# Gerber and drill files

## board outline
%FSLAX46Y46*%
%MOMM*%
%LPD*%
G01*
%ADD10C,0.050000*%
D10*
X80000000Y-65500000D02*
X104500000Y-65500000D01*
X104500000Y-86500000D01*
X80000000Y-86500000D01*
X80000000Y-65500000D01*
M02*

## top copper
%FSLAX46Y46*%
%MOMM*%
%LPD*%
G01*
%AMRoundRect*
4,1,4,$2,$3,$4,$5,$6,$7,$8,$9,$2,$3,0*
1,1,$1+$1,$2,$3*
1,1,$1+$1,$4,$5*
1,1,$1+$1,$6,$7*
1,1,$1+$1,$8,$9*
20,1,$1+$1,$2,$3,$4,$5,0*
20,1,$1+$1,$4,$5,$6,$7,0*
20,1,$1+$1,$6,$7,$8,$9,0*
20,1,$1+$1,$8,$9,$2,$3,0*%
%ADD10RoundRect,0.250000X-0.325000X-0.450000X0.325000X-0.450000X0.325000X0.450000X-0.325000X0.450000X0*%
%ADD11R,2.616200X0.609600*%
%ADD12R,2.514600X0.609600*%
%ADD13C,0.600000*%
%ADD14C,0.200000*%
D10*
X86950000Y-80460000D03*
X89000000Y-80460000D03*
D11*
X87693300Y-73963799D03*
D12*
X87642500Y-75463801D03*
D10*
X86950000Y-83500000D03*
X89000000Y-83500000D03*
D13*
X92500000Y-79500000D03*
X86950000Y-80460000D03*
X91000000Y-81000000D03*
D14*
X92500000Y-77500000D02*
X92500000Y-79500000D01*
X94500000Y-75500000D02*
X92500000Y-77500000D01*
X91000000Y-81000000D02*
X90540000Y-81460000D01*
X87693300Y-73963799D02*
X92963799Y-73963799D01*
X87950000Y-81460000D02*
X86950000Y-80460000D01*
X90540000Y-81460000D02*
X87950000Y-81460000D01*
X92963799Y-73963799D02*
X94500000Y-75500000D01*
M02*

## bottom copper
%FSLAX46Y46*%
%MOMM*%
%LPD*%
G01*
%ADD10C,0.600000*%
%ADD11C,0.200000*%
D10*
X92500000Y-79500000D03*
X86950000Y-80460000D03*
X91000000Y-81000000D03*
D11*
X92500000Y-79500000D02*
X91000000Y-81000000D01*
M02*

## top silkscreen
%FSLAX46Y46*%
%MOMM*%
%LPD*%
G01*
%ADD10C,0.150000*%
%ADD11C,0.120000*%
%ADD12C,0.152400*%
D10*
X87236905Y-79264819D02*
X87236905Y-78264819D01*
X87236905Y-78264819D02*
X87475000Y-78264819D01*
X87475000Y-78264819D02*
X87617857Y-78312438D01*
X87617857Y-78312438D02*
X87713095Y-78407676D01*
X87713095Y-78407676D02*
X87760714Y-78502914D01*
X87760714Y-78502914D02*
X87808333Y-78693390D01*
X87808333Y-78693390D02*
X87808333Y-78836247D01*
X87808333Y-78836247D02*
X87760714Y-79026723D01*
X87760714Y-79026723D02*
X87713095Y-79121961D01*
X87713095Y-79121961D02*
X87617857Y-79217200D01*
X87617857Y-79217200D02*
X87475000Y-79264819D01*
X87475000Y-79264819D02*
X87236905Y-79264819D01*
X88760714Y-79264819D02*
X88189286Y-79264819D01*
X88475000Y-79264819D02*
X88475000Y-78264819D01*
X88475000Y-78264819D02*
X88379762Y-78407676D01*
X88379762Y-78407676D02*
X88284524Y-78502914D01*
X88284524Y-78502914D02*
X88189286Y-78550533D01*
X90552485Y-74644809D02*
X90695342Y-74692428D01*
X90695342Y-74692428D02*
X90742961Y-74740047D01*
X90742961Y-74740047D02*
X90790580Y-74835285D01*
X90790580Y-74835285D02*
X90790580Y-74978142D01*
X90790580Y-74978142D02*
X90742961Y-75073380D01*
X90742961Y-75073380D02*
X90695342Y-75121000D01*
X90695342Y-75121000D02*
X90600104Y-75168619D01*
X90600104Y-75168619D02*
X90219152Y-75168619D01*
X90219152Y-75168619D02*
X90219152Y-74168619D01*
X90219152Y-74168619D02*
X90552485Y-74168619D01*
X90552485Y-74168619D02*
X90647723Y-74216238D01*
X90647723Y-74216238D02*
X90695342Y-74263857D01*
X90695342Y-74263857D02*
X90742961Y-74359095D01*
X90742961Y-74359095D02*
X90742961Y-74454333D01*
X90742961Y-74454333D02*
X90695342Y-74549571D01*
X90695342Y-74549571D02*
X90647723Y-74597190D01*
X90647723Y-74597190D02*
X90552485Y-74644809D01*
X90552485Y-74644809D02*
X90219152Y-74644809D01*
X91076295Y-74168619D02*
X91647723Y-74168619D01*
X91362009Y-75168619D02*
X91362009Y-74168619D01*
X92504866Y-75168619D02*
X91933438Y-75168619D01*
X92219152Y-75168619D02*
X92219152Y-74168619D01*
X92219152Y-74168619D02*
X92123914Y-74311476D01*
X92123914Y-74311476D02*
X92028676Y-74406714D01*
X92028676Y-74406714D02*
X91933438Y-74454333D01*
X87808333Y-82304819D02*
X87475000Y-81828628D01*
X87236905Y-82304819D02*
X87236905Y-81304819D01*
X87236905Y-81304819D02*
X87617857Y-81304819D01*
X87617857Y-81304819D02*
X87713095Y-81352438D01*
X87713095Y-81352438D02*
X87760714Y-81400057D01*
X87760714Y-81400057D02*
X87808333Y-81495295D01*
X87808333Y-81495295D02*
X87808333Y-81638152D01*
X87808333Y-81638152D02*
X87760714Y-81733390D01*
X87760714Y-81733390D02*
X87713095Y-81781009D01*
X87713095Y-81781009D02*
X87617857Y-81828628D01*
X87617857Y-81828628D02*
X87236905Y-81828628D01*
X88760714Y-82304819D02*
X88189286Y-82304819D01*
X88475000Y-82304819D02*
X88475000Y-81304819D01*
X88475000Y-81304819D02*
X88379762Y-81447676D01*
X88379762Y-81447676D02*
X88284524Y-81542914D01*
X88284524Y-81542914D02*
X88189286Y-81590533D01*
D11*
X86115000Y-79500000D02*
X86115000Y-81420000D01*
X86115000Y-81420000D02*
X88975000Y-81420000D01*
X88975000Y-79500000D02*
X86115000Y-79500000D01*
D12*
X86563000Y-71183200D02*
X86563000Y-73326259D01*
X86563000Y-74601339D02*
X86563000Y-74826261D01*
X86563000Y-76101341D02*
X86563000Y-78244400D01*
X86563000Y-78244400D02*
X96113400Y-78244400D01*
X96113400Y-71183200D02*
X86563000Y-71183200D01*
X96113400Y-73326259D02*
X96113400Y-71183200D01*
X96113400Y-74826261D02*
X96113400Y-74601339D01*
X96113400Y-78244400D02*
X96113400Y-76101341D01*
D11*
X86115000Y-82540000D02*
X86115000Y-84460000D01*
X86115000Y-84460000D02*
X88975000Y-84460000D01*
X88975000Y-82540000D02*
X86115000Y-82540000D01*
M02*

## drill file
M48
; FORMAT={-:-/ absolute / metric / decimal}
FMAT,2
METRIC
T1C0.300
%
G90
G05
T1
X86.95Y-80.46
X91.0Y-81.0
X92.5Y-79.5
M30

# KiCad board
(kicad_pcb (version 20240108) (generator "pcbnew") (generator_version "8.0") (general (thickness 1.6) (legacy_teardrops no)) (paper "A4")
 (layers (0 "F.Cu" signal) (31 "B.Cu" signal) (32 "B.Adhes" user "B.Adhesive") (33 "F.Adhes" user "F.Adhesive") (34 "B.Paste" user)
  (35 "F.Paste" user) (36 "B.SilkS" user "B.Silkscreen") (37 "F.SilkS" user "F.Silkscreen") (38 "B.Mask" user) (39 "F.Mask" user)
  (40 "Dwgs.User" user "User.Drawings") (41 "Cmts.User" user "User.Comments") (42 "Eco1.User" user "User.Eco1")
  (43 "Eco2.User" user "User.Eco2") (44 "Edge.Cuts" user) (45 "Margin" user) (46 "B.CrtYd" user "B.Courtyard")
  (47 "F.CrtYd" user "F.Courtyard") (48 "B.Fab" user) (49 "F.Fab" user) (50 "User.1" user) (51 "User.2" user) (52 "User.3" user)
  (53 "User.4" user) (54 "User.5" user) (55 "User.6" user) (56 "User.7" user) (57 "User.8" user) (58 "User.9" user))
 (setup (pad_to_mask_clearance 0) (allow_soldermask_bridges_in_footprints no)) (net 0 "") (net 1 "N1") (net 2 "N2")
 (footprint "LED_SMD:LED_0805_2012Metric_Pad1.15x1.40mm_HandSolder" (layer "F.Cu") (at 87.975 80.46)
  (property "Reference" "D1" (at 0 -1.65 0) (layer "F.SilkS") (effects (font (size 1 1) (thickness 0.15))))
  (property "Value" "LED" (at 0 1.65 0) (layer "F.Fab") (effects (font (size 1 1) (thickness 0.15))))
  (fp_line (start -1.86 -0.96) (end -1.86 0.96) (stroke (width 0.12) (type solid)) (layer "F.SilkS"))
  (fp_line (start -1.86 0.96) (end 1 0.96) (stroke (width 0.12) (type solid)) (layer "F.SilkS"))
  (fp_line (start 1 -0.96) (end -1.86 -0.96) (stroke (width 0.12) (type solid)) (layer "F.SilkS"))
  (pad "1" smd roundrect (at -1.025 0) (size 1.15 1.4) (layers "F.Cu" "F.Paste" "F.Mask") (roundrect_rratio 0.217391) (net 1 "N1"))
  (pad "2" smd roundrect (at 1.025 0) (size 1.15 1.4) (layers "F.Cu" "F.Paste" "F.Mask") (roundrect_rratio 0.217391) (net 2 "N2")))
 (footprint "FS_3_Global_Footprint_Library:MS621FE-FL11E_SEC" (layer "F.Cu") (at 91.3382 74.7138)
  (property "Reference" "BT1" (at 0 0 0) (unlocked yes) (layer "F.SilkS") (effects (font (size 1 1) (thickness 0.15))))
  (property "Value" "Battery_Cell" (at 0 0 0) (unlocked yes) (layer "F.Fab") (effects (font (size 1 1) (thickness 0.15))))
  (fp_line (start -4.7752 -3.5306) (end -4.7752 -1.387541) (stroke (width 0.1524) (type solid)) (layer "F.SilkS"))
  (fp_line (start -4.7752 -0.112461) (end -4.7752 0.112461) (stroke (width 0.1524) (type solid)) (layer "F.SilkS"))
  (fp_line (start -4.7752 1.387541) (end -4.7752 3.5306) (stroke (width 0.1524) (type solid)) (layer "F.SilkS"))
  (fp_line (start -4.7752 3.5306) (end 4.7752 3.5306) (stroke (width 0.1524) (type solid)) (layer "F.SilkS"))
  (fp_line (start 4.7752 -3.5306) (end -4.7752 -3.5306) (stroke (width 0.1524) (type solid)) (layer "F.SilkS"))
  (fp_line (start 4.7752 -1.387541) (end 4.7752 -3.5306) (stroke (width 0.1524) (type solid)) (layer "F.SilkS"))
  (fp_line (start 4.7752 0.112461) (end 4.7752 -0.112461) (stroke (width 0.1524) (type solid)) (layer "F.SilkS"))
  (fp_line (start 4.7752 3.5306) (end 4.7752 1.387541) (stroke (width 0.1524) (type solid)) (layer "F.SilkS"))
  (pad "1" smd rect (at -3.6449 -0.750001) (size 2.6162 0.6096) (layers "F.Cu" "F.Paste" "F.Mask") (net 1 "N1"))
  (pad "2" smd rect (at -3.6957 0.750001) (size 2.5146 0.6096) (layers "F.Cu" "F.Paste" "F.Mask") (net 1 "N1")))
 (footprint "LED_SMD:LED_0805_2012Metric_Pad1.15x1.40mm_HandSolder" (layer "F.Cu") (at 87.975 83.5)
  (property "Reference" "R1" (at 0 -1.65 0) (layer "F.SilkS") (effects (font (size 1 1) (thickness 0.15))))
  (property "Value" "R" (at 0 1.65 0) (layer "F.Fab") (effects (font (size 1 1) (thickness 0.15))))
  (fp_line (start -1.86 -0.96) (end -1.86 0.96) (stroke (width 0.12) (type solid)) (layer "F.SilkS"))
  (fp_line (start -1.86 0.96) (end 1 0.96) (stroke (width 0.12) (type solid)) (layer "F.SilkS"))
  (fp_line (start 1 -0.96) (end -1.86 -0.96) (stroke (width 0.12) (type solid)) (layer "F.SilkS"))
  (pad "1" smd roundrect (at -1.025 0) (size 1.15 1.4) (layers "F.Cu" "F.Paste" "F.Mask") (roundrect_rratio 0.217391) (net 1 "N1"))
  (pad "2" smd roundrect (at 1.025 0) (size 1.15 1.4) (layers "F.Cu" "F.Paste" "F.Mask") (roundrect_rratio 0.217391) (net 2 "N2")))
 (gr_rect (start 80 65.5) (end 104.5 86.5) (stroke (width 0.05) (type default)) (fill none) (layer "Edge.Cuts"))
 (segment (start 92.5 77.5) (end 92.5 79.5) (width 0.2) (layer "F.Cu") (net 1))
 (segment (start 94.5 75.5) (end 92.5 77.5) (width 0.2) (layer "F.Cu") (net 1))
 (segment (start 91 81) (end 90.54 81.46) (width 0.2) (layer "F.Cu") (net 1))
 (segment (start 87.6933 73.963799) (end 92.963799 73.963799) (width 0.2) (layer "F.Cu") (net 1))
 (segment (start 87.95 81.46) (end 86.95 80.46) (width 0.2) (layer "F.Cu") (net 1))
 (segment (start 90.54 81.46) (end 87.95 81.46) (width 0.2) (layer "F.Cu") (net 1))
 (segment (start 92.963799 73.963799) (end 94.5 75.5) (width 0.2) (layer "F.Cu") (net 1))
 (via (at 92.5 79.5) (size 0.6) (drill 0.3) (layers "F.Cu" "B.Cu") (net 1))
 (via (at 86.95 80.46) (size 0.6) (drill 0.3) (layers "F.Cu" "B.Cu") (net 1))
 (via (at 91 81) (size 0.6) (drill 0.3) (layers "F.Cu" "B.Cu") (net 1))
 (segment (start 92.5 79.5) (end 91 81) (width 0.2) (layer "B.Cu") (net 1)))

